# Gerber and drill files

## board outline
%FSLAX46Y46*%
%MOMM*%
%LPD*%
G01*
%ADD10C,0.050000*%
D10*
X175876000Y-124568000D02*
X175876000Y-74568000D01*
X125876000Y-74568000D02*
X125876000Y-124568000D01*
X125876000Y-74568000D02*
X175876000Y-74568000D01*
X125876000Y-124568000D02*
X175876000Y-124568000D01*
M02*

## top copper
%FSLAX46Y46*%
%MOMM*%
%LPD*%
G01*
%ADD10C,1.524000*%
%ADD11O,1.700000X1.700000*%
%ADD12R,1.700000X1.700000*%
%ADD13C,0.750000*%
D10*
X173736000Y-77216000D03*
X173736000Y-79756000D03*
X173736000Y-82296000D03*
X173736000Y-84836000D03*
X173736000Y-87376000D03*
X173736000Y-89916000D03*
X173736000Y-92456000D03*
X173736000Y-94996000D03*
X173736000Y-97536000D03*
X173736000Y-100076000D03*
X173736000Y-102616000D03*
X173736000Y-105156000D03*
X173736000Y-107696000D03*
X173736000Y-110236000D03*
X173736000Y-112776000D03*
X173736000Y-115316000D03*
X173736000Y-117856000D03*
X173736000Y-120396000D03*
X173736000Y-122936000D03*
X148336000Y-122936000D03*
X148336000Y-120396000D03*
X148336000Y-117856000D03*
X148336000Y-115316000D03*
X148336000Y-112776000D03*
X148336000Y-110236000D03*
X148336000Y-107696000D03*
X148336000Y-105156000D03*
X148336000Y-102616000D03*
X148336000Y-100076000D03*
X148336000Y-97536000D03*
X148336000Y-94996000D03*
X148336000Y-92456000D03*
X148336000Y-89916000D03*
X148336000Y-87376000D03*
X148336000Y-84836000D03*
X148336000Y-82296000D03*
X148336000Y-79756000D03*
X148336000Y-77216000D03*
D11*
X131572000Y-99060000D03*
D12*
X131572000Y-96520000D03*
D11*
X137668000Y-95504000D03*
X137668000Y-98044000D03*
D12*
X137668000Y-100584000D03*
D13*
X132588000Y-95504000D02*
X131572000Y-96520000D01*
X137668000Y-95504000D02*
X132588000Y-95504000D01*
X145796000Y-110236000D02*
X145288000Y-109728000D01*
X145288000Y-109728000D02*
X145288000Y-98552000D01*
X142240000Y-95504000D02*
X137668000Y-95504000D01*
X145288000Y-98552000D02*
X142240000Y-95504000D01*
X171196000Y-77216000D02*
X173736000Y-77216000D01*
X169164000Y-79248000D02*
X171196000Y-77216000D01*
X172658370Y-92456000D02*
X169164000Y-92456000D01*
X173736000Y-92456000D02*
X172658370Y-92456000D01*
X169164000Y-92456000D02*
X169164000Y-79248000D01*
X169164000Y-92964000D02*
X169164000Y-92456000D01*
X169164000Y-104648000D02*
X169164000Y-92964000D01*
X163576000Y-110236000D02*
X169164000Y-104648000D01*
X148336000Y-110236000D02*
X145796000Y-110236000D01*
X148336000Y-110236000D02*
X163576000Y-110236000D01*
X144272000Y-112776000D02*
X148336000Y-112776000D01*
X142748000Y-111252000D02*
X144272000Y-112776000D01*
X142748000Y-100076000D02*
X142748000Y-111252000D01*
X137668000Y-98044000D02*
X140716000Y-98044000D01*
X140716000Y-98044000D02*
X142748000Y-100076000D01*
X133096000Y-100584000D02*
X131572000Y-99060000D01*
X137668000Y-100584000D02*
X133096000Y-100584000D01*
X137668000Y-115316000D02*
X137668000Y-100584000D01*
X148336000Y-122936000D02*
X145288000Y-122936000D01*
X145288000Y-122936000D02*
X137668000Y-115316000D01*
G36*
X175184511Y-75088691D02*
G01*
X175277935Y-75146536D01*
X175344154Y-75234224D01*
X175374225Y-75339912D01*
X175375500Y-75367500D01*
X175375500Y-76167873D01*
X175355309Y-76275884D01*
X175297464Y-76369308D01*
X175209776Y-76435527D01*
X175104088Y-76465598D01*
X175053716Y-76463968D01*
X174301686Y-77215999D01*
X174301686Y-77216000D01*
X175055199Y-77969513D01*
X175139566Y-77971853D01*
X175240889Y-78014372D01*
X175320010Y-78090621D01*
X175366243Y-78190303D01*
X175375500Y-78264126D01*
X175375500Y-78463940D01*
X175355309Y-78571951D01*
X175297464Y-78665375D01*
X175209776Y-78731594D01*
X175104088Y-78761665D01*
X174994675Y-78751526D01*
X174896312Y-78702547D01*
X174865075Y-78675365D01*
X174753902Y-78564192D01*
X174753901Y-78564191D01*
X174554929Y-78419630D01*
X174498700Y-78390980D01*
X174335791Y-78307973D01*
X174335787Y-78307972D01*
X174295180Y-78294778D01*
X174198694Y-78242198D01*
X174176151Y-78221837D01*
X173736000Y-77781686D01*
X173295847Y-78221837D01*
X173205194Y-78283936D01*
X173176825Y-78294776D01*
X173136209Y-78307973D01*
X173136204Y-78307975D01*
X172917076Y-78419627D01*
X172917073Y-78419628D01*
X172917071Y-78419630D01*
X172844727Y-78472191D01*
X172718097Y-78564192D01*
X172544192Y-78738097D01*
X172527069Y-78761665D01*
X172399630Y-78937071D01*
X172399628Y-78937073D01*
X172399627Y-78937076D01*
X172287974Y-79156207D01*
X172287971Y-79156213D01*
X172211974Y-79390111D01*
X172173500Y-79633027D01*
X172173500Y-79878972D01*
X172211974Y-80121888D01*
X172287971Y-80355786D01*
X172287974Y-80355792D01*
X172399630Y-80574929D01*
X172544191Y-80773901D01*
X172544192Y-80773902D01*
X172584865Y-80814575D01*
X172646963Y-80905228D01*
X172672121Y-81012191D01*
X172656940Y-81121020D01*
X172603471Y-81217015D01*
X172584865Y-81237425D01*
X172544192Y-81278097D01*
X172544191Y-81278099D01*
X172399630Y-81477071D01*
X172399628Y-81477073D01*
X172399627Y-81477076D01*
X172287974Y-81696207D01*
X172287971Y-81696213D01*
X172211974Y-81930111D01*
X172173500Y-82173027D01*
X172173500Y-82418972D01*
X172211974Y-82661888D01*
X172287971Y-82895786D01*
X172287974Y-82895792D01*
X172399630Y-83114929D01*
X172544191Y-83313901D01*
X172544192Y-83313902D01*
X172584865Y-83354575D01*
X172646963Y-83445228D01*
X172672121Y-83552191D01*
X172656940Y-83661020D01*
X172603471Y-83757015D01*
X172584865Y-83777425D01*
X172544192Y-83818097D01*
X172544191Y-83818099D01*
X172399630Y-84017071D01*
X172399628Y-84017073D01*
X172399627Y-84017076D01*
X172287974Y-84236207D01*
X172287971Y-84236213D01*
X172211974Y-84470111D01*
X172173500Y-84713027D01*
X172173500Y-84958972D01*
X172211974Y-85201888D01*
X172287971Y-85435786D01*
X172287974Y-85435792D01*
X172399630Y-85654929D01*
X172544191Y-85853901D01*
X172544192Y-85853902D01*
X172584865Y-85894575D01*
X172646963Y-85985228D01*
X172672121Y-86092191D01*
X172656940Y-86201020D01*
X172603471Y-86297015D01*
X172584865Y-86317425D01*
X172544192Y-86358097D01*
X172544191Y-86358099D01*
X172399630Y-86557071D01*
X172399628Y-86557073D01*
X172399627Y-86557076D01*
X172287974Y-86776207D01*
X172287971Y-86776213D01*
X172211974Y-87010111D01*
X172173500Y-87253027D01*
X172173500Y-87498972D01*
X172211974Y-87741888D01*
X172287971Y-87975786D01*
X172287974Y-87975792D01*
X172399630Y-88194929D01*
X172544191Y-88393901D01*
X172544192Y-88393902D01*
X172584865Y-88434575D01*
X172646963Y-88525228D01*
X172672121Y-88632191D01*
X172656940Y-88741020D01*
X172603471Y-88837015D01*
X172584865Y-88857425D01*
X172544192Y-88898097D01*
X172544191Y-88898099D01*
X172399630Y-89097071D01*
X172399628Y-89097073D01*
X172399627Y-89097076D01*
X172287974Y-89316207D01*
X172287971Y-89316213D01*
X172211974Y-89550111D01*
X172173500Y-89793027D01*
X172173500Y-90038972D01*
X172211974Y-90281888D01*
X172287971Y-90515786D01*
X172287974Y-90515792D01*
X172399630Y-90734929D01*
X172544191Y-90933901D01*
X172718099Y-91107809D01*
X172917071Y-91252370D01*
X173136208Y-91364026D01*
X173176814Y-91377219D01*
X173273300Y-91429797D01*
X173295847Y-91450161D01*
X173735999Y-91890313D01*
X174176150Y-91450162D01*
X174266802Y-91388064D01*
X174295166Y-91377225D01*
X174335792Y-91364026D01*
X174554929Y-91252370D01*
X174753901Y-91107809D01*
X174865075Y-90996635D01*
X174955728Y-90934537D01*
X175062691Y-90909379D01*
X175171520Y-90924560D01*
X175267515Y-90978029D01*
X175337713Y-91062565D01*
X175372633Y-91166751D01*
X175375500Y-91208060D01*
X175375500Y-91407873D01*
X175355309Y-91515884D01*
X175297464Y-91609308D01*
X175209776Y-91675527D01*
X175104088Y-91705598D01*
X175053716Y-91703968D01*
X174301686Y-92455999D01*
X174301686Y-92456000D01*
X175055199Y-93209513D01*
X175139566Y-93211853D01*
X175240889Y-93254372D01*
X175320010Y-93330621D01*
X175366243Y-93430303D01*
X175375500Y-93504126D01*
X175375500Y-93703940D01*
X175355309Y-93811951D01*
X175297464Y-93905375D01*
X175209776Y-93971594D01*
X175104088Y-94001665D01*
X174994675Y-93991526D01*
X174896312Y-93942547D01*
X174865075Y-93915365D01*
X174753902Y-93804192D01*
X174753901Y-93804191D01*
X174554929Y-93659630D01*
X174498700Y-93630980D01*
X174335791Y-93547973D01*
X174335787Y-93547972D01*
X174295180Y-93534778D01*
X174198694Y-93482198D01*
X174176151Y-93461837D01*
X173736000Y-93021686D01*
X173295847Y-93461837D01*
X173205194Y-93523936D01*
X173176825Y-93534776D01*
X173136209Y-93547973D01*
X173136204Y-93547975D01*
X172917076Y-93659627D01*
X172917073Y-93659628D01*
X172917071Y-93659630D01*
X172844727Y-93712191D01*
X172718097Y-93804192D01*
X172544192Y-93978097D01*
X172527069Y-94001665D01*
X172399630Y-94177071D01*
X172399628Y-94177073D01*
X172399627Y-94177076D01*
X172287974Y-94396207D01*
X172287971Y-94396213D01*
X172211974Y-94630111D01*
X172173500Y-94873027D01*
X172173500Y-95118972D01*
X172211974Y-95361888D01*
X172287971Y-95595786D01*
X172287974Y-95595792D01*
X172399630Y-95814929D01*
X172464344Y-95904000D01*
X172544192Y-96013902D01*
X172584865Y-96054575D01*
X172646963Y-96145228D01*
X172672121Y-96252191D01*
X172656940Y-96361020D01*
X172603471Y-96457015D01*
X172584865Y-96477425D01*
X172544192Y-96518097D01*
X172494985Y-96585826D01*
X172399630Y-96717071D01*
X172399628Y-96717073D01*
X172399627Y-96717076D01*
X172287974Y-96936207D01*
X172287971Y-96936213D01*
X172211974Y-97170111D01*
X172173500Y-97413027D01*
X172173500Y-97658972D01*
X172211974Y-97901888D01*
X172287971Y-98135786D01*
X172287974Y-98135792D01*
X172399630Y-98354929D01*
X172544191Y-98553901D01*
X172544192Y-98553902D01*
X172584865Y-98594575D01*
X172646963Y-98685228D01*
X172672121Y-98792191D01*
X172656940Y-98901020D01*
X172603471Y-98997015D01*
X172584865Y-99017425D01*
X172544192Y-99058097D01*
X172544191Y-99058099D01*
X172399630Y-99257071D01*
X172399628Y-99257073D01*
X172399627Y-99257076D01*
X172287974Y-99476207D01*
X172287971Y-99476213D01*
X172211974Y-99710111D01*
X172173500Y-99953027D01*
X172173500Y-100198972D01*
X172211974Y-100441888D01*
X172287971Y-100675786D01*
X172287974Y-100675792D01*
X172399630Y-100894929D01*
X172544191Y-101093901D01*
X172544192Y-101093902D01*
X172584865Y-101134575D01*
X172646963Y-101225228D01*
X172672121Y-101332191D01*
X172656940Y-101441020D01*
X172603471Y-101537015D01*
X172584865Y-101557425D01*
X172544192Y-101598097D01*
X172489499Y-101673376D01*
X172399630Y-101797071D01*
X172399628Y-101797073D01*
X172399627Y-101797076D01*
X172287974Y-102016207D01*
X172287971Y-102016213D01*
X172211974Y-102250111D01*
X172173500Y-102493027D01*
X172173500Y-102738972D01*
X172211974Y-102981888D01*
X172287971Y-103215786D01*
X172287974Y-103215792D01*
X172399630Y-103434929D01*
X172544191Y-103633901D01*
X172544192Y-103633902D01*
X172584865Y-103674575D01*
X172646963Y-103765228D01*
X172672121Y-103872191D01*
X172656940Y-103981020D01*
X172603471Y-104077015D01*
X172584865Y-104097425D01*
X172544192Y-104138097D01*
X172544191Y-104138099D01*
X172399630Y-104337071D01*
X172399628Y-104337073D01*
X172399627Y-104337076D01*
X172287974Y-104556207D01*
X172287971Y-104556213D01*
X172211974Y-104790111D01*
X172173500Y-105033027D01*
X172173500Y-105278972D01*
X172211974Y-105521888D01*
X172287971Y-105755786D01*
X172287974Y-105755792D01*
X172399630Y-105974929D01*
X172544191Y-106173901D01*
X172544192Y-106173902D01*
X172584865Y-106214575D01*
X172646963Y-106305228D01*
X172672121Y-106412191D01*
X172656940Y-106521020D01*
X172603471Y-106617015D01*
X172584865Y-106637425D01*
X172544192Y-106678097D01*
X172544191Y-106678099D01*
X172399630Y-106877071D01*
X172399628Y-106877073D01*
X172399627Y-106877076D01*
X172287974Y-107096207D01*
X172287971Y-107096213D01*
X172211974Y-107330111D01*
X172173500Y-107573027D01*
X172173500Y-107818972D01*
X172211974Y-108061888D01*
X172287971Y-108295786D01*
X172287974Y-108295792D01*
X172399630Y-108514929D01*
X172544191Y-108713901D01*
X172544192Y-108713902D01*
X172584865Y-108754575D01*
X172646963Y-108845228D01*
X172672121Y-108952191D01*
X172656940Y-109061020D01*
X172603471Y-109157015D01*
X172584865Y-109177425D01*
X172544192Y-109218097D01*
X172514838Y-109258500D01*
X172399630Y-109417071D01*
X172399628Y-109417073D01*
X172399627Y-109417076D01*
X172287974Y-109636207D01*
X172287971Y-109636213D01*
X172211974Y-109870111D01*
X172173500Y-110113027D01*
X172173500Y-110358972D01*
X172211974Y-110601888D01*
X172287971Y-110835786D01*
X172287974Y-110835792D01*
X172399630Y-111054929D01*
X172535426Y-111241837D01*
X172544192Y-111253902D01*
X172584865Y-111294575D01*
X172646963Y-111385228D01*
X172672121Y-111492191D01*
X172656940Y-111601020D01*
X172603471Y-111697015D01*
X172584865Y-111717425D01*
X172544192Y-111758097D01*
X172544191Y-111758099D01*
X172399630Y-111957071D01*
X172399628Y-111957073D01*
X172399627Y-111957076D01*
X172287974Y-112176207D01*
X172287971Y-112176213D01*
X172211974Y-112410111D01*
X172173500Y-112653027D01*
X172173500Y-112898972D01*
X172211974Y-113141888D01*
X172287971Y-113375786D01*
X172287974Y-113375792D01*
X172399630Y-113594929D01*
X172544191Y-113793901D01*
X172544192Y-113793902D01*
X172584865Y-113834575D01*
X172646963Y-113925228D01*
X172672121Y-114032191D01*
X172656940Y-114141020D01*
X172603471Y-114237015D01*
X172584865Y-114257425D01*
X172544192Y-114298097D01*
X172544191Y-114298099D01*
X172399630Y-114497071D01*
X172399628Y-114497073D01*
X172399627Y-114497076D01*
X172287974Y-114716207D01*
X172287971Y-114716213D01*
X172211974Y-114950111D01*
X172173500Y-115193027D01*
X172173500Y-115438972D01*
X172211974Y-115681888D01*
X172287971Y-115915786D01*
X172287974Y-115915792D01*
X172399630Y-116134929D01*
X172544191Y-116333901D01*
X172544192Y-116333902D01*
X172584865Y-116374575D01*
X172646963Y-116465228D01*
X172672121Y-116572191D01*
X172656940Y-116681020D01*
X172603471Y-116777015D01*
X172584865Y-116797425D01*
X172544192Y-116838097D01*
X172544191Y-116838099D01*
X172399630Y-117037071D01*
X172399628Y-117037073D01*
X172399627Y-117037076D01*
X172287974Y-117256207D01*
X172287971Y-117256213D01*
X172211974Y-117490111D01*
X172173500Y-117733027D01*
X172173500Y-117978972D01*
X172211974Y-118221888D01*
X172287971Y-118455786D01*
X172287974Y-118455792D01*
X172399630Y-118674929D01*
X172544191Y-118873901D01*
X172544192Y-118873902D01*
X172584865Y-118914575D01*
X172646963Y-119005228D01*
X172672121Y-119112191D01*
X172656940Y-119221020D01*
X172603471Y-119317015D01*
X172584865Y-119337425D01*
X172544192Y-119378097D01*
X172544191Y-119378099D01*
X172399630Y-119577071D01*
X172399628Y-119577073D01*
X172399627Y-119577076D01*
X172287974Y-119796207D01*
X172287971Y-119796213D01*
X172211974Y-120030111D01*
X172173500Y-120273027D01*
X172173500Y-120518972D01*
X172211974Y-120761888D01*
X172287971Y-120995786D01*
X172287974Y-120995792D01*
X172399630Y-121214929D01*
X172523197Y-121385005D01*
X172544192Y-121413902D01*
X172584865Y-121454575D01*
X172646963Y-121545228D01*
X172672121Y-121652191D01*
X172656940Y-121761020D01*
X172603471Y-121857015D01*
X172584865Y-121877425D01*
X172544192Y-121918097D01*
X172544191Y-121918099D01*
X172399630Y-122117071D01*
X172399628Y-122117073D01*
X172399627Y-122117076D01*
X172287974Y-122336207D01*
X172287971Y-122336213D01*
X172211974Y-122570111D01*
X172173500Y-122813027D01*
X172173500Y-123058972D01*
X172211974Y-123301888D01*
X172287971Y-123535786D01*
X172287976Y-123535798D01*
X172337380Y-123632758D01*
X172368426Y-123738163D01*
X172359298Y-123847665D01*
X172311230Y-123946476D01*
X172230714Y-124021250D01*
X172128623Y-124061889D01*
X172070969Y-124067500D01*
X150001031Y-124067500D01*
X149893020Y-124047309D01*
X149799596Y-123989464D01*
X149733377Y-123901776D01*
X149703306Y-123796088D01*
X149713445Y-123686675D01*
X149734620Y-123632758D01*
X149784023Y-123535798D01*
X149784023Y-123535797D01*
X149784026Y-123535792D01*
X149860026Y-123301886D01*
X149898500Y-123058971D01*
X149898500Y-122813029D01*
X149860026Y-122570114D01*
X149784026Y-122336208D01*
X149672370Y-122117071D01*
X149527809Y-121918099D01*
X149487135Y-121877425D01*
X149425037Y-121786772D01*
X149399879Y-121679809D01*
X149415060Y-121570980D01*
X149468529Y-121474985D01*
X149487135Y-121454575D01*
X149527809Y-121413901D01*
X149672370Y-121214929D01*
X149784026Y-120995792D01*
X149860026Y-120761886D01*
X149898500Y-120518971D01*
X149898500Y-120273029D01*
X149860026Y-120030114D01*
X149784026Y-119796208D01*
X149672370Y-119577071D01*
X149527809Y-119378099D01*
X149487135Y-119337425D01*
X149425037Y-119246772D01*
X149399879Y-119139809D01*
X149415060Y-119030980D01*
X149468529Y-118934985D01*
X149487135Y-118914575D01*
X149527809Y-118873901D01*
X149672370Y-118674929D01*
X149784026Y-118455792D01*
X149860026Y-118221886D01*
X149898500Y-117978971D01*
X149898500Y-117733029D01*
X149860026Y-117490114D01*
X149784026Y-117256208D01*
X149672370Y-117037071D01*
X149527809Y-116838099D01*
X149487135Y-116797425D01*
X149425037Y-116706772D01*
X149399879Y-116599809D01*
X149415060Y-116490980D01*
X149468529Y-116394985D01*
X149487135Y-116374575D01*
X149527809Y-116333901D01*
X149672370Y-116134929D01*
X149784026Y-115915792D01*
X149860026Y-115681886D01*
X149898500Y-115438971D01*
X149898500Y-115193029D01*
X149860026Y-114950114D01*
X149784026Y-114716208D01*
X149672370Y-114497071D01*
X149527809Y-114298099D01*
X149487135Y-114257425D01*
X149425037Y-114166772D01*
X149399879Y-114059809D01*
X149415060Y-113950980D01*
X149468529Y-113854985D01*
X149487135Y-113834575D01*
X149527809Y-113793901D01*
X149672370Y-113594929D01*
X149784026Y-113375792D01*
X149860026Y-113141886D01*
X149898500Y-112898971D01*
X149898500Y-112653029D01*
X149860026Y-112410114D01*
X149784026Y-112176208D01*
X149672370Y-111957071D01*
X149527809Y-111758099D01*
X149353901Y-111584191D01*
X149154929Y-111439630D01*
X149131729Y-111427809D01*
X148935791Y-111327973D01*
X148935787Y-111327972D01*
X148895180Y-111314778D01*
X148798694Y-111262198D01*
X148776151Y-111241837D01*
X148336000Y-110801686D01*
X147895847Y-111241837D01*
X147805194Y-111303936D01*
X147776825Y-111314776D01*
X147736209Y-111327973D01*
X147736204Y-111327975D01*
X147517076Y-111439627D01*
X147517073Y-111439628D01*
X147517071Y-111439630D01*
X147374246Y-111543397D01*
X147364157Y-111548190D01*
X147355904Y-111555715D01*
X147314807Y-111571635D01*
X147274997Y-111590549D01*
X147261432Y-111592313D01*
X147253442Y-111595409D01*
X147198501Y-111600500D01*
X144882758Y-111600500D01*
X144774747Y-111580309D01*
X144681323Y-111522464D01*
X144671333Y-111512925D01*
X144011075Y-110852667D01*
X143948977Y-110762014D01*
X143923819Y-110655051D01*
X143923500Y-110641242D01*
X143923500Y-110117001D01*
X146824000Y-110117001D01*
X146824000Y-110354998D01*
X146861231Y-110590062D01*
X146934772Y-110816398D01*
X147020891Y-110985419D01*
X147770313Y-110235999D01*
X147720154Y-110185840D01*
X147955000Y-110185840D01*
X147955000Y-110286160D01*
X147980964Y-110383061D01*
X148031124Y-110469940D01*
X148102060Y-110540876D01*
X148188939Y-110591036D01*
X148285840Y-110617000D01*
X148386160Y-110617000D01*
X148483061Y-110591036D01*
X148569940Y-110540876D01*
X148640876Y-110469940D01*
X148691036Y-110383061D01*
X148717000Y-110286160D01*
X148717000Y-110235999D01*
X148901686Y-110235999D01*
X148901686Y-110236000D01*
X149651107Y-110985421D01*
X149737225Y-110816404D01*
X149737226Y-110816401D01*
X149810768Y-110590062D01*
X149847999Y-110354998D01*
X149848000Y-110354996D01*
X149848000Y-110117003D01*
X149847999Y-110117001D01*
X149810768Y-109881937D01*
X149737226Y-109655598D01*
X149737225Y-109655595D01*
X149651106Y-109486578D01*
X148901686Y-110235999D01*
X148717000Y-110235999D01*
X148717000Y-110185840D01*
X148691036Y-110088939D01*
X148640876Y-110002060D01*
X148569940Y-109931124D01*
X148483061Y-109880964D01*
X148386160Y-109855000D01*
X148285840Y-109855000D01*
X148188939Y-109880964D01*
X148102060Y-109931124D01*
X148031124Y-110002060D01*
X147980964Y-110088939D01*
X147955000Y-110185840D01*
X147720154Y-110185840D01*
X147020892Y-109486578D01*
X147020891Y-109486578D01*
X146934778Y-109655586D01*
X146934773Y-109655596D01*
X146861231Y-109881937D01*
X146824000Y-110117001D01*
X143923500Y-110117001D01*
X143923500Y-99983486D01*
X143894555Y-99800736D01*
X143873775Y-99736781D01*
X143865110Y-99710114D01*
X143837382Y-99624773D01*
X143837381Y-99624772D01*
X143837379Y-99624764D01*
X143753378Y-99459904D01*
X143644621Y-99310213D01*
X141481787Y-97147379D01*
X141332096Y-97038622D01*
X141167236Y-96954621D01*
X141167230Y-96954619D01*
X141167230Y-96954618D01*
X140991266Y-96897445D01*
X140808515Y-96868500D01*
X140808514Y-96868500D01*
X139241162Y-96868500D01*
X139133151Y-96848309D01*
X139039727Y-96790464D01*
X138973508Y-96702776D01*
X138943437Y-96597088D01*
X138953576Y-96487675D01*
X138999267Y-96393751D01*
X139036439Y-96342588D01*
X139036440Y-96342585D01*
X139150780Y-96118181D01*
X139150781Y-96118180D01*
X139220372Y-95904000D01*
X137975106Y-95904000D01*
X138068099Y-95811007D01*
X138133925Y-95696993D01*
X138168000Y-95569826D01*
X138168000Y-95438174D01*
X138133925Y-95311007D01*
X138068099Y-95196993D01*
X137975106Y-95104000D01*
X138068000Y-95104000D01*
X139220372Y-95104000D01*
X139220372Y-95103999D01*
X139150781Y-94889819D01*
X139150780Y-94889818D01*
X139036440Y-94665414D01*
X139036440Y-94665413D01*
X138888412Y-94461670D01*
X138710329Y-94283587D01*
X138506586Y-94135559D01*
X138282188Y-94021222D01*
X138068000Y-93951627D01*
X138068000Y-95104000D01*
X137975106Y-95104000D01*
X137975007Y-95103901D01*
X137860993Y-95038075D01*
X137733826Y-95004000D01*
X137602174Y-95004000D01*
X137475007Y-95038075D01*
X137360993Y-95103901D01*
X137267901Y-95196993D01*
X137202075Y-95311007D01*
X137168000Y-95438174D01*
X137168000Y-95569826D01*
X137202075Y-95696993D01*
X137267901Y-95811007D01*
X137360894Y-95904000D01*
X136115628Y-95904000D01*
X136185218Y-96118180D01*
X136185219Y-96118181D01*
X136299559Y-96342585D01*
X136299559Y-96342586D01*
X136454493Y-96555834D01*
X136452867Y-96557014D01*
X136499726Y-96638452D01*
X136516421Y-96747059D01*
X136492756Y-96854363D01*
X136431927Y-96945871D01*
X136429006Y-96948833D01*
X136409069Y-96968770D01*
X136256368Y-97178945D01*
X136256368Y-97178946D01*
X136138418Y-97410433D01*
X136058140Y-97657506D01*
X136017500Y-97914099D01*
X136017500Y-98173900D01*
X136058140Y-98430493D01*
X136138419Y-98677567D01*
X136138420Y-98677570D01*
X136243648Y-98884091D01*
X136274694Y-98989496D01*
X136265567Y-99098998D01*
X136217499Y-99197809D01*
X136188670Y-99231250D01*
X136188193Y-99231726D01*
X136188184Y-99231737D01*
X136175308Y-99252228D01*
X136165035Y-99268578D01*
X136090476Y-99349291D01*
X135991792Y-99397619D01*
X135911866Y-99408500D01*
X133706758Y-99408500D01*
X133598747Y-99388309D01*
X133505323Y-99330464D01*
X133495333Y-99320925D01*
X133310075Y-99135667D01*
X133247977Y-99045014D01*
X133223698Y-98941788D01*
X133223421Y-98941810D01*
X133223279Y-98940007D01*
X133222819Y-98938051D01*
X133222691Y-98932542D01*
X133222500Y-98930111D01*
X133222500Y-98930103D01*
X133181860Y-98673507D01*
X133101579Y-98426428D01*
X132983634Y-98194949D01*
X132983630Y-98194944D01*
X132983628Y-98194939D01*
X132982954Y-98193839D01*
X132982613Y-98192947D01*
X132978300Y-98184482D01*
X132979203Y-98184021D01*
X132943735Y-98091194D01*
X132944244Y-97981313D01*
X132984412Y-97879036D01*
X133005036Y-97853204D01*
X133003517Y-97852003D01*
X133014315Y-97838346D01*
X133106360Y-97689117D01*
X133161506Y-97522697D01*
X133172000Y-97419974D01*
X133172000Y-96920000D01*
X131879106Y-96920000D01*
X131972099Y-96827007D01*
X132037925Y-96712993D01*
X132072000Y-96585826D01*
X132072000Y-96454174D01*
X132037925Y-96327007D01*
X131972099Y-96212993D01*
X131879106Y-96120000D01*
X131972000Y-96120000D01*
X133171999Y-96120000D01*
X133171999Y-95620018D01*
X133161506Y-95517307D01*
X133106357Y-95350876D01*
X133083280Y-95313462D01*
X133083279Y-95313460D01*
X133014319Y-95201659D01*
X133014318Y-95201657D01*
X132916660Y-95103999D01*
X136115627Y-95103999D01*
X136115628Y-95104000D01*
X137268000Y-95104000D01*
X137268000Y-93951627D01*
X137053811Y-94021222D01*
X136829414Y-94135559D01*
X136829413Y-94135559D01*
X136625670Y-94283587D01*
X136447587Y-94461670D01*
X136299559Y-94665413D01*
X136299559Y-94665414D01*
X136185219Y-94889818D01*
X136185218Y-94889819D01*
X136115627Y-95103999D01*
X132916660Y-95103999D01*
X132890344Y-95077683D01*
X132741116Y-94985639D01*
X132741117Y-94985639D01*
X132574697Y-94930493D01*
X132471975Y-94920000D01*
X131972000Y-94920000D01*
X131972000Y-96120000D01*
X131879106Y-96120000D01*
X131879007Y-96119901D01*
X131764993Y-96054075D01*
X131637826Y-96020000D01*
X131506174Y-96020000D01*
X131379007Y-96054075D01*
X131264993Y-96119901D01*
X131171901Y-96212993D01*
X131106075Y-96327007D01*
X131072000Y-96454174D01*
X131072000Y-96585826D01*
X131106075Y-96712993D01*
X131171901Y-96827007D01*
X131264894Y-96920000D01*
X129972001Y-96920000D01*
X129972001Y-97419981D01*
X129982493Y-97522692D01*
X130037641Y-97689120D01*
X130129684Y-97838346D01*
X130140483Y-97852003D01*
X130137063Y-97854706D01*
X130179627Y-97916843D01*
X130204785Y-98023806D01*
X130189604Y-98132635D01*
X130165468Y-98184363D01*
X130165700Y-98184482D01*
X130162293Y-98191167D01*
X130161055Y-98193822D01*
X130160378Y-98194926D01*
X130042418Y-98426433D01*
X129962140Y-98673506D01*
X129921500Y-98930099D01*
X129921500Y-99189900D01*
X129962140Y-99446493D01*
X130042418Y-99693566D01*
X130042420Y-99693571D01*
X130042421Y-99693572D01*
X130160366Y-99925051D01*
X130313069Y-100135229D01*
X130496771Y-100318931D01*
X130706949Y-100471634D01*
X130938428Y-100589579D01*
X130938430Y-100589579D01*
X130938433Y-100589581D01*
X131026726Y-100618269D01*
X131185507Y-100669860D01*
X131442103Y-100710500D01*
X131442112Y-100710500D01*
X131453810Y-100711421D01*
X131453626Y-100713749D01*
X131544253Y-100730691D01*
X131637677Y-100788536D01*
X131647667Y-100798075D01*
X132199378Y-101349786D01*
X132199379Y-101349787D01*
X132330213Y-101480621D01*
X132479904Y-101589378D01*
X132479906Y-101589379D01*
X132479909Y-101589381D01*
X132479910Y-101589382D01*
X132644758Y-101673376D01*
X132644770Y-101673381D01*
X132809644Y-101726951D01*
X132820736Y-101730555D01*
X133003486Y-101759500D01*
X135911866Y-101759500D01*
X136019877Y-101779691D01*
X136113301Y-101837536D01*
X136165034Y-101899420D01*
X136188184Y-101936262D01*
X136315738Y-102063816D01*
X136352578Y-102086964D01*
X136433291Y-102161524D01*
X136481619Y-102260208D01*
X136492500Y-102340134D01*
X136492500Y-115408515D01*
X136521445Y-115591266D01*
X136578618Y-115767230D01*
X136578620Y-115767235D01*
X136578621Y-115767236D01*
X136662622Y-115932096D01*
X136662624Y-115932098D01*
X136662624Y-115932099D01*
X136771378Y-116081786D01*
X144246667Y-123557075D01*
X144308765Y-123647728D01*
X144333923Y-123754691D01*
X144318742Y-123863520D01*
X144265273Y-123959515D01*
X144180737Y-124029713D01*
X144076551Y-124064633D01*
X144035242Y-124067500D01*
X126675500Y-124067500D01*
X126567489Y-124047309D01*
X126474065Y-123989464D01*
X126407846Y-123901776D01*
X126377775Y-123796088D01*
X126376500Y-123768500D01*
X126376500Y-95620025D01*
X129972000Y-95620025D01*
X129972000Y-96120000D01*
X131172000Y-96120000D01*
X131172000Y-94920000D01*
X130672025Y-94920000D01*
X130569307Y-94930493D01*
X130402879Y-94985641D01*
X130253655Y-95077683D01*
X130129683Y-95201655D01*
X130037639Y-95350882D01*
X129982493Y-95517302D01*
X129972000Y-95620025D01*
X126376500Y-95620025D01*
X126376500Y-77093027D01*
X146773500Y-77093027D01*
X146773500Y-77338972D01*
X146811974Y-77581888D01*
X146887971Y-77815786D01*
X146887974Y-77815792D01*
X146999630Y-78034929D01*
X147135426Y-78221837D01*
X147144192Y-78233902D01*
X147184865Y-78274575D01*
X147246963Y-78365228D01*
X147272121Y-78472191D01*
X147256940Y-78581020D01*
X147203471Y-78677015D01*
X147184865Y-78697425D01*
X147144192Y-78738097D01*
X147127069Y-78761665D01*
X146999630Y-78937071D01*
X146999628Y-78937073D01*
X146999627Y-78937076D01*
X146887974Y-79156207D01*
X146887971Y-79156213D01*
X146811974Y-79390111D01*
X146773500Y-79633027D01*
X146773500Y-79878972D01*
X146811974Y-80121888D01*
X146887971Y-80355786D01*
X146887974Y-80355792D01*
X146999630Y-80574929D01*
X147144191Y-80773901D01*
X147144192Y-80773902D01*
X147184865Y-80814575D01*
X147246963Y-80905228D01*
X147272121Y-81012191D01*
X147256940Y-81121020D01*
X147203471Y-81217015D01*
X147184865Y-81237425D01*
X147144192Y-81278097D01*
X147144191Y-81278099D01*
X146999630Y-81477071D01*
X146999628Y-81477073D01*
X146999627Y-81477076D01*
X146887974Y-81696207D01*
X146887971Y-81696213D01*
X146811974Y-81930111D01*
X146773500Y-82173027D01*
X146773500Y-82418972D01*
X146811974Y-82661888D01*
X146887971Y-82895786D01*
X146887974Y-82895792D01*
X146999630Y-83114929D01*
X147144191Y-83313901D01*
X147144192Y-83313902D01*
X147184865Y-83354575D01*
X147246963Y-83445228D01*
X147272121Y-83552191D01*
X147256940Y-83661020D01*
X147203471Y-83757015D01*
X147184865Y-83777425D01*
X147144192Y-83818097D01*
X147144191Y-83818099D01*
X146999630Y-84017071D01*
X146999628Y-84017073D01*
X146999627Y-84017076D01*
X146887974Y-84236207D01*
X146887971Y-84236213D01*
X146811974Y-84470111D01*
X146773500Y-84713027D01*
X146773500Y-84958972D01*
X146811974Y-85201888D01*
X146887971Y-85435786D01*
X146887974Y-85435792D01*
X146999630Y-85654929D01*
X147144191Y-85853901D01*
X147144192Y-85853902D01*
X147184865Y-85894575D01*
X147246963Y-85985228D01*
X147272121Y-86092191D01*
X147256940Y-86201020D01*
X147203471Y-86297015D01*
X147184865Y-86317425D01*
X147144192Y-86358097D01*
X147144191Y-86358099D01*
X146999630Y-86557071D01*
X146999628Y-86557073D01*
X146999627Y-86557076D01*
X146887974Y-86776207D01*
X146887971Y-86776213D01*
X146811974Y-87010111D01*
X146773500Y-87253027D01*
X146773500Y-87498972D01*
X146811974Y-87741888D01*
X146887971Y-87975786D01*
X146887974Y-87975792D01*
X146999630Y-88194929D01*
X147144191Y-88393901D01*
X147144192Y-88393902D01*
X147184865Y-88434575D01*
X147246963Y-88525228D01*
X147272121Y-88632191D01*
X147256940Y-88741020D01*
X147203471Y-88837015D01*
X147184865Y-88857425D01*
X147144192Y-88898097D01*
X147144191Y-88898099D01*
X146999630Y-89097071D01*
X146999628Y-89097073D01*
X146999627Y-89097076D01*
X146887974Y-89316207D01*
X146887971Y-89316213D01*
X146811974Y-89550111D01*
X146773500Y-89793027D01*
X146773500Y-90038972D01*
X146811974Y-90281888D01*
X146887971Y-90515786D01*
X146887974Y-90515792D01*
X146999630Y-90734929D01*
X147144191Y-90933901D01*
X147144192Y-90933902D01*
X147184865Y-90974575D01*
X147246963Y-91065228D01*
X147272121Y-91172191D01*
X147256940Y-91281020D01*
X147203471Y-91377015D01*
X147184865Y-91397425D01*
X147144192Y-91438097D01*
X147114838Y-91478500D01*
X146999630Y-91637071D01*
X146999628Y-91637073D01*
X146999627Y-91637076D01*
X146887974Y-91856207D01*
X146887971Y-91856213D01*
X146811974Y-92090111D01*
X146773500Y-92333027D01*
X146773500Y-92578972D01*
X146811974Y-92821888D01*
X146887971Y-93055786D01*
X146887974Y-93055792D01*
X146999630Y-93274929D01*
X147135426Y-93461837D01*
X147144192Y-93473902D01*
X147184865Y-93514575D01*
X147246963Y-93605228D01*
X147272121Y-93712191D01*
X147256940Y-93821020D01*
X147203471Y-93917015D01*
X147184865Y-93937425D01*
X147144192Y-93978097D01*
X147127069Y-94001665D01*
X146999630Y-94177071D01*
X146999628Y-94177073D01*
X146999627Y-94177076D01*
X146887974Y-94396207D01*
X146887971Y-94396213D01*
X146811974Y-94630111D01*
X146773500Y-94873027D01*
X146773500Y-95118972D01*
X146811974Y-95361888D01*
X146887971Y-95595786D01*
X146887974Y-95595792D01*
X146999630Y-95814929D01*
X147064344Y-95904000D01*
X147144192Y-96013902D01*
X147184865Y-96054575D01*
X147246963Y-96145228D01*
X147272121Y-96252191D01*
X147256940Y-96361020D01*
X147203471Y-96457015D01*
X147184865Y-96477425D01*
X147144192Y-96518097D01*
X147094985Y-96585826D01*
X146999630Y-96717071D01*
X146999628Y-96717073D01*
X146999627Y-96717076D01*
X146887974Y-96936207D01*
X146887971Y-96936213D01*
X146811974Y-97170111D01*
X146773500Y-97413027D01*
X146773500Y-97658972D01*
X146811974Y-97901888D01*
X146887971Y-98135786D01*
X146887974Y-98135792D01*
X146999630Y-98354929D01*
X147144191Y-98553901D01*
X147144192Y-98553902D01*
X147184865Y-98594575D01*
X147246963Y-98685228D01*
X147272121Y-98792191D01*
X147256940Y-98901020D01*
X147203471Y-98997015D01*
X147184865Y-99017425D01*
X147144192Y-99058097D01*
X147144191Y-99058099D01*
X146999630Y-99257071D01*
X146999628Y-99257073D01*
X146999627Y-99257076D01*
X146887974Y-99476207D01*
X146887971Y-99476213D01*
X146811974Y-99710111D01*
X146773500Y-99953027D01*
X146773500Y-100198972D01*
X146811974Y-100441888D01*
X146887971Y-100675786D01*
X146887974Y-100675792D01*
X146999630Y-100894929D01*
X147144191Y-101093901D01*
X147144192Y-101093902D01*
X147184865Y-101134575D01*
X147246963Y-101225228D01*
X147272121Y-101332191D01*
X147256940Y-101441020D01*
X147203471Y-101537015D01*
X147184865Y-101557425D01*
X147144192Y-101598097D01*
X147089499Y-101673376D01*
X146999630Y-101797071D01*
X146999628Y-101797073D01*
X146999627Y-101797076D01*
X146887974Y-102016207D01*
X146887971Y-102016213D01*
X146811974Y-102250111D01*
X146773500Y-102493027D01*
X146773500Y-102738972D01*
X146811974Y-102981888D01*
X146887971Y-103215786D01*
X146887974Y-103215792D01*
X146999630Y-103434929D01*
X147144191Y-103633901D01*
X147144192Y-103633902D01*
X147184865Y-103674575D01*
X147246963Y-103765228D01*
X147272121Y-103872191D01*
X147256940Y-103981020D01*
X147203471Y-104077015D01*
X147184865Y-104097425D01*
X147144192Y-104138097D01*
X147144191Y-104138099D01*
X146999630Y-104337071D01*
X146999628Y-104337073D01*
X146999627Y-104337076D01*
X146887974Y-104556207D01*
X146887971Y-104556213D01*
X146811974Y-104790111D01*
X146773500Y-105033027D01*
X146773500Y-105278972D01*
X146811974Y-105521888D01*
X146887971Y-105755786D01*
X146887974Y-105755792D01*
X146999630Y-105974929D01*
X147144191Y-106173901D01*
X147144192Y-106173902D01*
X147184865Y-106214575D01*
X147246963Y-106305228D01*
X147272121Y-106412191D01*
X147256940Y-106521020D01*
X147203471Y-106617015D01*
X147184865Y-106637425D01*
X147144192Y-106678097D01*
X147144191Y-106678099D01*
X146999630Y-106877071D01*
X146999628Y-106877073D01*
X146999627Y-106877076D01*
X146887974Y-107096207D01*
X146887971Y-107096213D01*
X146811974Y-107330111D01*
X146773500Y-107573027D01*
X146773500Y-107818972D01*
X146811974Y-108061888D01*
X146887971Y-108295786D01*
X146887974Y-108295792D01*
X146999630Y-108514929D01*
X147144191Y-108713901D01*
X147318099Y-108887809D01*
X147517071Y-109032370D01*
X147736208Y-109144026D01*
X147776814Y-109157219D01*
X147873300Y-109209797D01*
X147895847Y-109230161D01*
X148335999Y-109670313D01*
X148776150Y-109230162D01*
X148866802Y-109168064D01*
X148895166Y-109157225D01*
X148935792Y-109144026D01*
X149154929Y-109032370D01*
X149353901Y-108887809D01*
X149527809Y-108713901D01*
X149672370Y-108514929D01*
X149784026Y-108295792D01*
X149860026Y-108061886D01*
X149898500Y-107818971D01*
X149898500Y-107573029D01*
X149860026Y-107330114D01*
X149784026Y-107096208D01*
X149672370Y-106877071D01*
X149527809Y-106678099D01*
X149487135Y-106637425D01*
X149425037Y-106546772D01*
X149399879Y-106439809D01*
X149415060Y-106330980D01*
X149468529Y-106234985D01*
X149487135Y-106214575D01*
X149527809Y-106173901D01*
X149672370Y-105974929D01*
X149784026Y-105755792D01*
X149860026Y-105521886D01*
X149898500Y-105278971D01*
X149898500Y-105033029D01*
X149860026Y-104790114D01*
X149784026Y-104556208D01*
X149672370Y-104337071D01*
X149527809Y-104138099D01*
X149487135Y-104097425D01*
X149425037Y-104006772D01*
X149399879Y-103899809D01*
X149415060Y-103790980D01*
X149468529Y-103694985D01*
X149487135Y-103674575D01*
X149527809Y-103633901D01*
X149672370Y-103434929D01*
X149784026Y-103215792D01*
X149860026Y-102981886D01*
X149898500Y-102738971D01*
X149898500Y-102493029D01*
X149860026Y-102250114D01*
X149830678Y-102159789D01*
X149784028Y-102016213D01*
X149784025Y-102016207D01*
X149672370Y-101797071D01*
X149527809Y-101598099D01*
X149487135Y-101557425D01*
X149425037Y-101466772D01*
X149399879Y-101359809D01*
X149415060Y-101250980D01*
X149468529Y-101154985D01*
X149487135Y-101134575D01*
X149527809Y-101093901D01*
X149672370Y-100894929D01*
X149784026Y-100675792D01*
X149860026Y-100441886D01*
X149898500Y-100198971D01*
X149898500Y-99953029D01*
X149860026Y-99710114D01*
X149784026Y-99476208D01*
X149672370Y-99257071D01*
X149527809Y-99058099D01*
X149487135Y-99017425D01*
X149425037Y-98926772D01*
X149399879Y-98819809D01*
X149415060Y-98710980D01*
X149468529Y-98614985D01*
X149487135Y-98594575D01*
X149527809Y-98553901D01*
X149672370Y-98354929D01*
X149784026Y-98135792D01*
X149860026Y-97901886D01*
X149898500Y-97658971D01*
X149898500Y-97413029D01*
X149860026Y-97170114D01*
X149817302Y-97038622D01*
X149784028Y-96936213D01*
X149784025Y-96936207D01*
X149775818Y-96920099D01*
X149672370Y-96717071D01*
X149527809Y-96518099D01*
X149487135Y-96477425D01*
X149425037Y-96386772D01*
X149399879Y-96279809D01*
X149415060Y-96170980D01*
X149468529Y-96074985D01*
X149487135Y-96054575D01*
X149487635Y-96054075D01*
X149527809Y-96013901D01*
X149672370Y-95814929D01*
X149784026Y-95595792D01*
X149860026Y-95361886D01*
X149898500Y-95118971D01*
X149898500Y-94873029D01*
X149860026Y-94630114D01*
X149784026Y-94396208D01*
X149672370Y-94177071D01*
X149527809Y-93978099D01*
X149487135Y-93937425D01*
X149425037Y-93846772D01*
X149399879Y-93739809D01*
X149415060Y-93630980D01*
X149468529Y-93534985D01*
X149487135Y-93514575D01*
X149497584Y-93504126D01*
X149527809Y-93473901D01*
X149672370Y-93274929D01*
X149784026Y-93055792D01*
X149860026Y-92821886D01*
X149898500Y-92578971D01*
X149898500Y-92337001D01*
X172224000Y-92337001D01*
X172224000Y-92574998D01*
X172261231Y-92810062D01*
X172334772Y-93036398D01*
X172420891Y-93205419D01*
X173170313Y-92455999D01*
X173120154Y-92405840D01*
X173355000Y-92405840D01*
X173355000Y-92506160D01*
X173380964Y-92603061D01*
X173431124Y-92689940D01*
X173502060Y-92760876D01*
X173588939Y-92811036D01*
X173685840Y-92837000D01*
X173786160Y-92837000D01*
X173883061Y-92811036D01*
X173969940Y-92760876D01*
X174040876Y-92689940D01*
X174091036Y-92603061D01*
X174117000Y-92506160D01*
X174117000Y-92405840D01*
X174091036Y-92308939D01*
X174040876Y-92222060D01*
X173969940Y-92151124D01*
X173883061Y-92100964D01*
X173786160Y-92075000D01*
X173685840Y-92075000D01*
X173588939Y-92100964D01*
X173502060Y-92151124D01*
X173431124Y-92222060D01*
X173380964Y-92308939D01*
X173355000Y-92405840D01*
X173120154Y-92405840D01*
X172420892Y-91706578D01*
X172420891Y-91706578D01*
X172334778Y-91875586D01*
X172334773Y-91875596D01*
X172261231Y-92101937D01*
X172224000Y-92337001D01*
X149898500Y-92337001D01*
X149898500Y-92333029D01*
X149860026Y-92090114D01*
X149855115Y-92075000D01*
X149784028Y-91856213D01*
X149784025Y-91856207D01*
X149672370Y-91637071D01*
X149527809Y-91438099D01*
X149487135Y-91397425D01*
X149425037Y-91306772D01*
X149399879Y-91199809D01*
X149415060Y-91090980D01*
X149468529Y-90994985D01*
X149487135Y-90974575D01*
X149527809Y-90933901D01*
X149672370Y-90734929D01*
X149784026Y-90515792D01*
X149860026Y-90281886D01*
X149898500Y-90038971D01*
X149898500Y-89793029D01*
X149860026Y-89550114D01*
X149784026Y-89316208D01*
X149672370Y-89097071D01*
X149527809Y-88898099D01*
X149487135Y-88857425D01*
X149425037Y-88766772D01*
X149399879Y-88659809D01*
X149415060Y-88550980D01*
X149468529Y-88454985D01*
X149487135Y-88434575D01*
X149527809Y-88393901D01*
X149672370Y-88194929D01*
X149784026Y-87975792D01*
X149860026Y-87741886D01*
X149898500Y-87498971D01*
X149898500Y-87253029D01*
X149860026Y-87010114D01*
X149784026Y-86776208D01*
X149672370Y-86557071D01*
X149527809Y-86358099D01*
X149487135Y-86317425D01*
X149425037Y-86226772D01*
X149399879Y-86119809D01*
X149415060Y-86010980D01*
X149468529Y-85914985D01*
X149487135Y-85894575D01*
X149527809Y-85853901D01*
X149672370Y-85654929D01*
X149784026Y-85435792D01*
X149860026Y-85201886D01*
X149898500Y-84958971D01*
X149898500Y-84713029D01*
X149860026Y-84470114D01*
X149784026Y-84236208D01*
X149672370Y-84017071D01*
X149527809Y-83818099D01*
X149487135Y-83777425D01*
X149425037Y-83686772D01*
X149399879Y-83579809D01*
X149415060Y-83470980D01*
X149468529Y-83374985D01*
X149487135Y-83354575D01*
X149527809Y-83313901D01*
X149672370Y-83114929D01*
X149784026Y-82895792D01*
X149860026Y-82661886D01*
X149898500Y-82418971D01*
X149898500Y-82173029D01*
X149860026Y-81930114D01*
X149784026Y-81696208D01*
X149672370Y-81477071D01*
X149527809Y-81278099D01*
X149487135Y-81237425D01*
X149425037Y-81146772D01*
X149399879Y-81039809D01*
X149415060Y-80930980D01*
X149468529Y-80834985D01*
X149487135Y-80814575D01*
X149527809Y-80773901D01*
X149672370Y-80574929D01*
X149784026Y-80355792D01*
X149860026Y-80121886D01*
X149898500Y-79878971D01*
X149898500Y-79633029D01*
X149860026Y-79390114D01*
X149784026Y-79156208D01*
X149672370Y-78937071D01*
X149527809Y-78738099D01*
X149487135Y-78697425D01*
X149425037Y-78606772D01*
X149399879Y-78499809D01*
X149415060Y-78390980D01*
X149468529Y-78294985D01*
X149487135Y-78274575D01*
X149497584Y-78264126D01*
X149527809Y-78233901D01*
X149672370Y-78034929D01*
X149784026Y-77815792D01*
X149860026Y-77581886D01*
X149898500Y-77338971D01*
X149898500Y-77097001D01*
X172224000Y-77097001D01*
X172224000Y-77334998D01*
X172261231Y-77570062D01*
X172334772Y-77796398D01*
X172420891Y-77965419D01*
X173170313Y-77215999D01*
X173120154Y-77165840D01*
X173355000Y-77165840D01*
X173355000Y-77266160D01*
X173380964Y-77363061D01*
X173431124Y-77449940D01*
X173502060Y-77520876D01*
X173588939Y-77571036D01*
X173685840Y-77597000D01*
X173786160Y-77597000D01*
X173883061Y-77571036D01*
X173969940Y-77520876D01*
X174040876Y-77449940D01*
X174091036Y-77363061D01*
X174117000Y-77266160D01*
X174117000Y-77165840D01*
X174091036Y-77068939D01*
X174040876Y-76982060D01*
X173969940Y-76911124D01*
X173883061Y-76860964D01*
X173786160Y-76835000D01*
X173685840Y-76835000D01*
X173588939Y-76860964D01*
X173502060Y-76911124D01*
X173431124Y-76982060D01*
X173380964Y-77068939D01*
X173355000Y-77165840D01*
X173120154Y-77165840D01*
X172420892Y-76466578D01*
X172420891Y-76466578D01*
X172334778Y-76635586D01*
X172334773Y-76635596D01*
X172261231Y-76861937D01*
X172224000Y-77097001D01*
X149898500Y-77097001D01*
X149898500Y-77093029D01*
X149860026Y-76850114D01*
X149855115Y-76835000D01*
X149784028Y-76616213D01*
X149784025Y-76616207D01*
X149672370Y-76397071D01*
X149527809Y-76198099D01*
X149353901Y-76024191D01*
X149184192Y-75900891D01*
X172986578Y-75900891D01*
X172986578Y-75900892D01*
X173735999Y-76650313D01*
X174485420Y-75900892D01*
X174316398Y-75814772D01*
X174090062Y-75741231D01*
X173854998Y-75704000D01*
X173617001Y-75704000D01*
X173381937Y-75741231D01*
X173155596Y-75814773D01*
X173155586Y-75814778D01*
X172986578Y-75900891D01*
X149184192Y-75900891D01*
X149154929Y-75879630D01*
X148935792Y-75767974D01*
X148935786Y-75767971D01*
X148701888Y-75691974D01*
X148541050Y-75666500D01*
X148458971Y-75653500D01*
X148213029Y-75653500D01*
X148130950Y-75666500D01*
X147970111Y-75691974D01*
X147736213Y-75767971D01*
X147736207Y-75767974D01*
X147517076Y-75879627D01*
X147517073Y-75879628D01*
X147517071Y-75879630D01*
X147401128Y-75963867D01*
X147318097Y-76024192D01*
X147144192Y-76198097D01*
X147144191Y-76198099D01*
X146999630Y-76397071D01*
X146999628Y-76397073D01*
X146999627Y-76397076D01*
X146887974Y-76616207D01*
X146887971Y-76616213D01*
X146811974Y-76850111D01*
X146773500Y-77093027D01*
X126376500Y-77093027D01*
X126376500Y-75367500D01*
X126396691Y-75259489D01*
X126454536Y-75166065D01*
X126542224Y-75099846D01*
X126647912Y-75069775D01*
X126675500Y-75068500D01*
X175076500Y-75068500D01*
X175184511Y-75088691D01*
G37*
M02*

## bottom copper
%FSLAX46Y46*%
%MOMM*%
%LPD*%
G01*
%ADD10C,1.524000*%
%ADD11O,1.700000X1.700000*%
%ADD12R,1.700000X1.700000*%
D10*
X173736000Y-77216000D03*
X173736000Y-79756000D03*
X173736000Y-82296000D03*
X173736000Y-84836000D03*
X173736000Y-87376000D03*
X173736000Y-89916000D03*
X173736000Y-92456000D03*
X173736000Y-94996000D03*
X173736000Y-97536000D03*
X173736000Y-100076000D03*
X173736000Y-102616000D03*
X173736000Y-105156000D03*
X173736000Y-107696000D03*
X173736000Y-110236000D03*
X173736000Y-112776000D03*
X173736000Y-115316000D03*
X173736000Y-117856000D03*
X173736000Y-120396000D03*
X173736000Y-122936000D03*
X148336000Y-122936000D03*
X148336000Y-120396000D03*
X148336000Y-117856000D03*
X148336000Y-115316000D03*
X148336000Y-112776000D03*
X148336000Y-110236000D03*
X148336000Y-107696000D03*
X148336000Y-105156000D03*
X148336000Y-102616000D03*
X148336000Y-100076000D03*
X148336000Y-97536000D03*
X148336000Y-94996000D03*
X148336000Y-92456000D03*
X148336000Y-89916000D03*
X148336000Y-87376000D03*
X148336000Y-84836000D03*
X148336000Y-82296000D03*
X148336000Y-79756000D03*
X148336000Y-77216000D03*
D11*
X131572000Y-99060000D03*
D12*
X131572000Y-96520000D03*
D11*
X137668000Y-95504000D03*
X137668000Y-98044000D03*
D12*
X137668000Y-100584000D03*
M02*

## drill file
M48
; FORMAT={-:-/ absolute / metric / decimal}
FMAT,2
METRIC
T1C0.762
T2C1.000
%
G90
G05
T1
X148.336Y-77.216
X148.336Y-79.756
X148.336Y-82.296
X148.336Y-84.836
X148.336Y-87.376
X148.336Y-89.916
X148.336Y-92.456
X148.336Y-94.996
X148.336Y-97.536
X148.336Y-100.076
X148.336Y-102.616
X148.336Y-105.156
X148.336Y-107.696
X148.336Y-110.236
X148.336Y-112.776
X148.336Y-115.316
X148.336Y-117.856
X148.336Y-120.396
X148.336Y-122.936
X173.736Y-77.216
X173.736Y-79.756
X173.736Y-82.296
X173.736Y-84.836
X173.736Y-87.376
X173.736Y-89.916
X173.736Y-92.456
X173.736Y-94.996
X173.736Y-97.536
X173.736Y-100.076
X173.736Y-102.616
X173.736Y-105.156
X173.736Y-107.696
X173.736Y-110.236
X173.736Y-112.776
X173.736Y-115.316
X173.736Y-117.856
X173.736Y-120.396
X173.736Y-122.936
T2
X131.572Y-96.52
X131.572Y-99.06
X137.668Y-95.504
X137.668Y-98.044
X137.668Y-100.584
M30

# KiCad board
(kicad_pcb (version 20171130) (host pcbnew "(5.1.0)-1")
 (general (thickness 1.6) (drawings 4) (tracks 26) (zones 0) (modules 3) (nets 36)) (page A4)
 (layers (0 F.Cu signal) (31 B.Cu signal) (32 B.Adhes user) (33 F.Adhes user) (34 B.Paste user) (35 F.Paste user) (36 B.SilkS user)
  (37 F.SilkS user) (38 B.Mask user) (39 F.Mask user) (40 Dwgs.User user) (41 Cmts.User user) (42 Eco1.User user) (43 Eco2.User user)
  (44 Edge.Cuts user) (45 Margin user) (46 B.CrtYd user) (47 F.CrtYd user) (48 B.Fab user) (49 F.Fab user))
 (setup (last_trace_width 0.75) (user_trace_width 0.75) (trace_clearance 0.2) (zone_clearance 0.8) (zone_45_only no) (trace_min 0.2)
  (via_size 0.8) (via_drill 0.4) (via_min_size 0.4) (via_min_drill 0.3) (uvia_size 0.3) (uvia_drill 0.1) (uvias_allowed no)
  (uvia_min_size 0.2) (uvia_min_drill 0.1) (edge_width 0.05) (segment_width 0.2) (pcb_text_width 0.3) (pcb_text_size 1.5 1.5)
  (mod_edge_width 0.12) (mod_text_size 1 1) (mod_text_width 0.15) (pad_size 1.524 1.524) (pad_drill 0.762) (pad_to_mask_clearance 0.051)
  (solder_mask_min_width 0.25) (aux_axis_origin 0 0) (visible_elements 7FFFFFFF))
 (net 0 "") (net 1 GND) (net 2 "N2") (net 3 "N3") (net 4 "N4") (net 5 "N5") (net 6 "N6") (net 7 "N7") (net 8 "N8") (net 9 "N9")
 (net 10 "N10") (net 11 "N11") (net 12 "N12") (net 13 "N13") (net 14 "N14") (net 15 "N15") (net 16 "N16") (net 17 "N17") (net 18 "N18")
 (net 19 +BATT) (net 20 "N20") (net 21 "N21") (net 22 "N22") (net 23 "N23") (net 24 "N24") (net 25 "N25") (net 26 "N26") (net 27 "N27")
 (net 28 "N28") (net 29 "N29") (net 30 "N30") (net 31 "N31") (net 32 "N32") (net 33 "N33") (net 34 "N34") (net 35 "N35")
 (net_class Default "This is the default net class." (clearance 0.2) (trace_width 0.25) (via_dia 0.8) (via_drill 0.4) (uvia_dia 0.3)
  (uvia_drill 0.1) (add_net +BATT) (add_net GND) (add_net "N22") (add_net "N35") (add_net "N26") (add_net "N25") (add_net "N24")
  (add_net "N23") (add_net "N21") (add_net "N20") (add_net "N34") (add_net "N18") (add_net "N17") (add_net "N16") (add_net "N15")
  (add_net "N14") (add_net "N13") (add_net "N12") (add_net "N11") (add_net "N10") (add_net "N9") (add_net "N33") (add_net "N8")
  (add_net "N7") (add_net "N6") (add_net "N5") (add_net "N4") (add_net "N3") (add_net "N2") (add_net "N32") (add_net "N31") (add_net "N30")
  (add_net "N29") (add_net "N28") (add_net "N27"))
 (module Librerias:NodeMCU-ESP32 (layer F.Cu) (at 161.036 97.536)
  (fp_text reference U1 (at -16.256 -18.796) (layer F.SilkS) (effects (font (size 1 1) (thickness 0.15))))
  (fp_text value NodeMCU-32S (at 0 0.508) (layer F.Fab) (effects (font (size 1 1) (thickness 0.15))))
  (pad 38 thru_hole circle (at 12.7 -20.32) (size 1.524 1.524) (drill 0.762) (layers *.Cu *.Mask) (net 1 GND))
  (pad 37 thru_hole circle (at 12.7 -17.78) (size 1.524 1.524) (drill 0.762) (layers *.Cu *.Mask) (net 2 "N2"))
  (pad 36 thru_hole circle (at 12.7 -15.24) (size 1.524 1.524) (drill 0.762) (layers *.Cu *.Mask) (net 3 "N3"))
  (pad 35 thru_hole circle (at 12.7 -12.7) (size 1.524 1.524) (drill 0.762) (layers *.Cu *.Mask) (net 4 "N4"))
  (pad 34 thru_hole circle (at 12.7 -10.16) (size 1.524 1.524) (drill 0.762) (layers *.Cu *.Mask) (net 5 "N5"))
  (pad 33 thru_hole circle (at 12.7 -7.62) (size 1.524 1.524) (drill 0.762) (layers *.Cu *.Mask) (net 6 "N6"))
  (pad 32 thru_hole circle (at 12.7 -5.08) (size 1.524 1.524) (drill 0.762) (layers *.Cu *.Mask) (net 1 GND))
  (pad 31 thru_hole circle (at 12.7 -2.54) (size 1.524 1.524) (drill 0.762) (layers *.Cu *.Mask) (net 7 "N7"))
  (pad 30 thru_hole circle (at 12.7 0) (size 1.524 1.524) (drill 0.762) (layers *.Cu *.Mask) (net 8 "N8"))
  (pad 29 thru_hole circle (at 12.7 2.54) (size 1.524 1.524) (drill 0.762) (layers *.Cu *.Mask) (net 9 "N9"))
  (pad 28 thru_hole circle (at 12.7 5.08) (size 1.524 1.524) (drill 0.762) (layers *.Cu *.Mask) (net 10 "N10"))
  (pad 27 thru_hole circle (at 12.7 7.62) (size 1.524 1.524) (drill 0.762) (layers *.Cu *.Mask) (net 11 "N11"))
  (pad 26 thru_hole circle (at 12.7 10.16) (size 1.524 1.524) (drill 0.762) (layers *.Cu *.Mask) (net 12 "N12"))
  (pad 25 thru_hole circle (at 12.7 12.7) (size 1.524 1.524) (drill 0.762) (layers *.Cu *.Mask) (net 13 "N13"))
  (pad 24 thru_hole circle (at 12.7 15.24) (size 1.524 1.524) (drill 0.762) (layers *.Cu *.Mask) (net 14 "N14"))
  (pad 23 thru_hole circle (at 12.7 17.78) (size 1.524 1.524) (drill 0.762) (layers *.Cu *.Mask) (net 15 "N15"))
  (pad 22 thru_hole circle (at 12.7 20.32) (size 1.524 1.524) (drill 0.762) (layers *.Cu *.Mask) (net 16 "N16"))
  (pad 21 thru_hole circle (at 12.7 22.86) (size 1.524 1.524) (drill 0.762) (layers *.Cu *.Mask) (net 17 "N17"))
  (pad 20 thru_hole circle (at 12.7 25.4) (size 1.524 1.524) (drill 0.762) (layers *.Cu *.Mask) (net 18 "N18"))
  (pad 19 thru_hole circle (at -12.7 25.4) (size 1.524 1.524) (drill 0.762) (layers *.Cu *.Mask) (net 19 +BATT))
  (pad 18 thru_hole circle (at -12.7 22.86) (size 1.524 1.524) (drill 0.762) (layers *.Cu *.Mask) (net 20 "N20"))
  (pad 17 thru_hole circle (at -12.7 20.32) (size 1.524 1.524) (drill 0.762) (layers *.Cu *.Mask) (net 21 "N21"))
  (pad 16 thru_hole circle (at -12.7 17.78) (size 1.524 1.524) (drill 0.762) (layers *.Cu *.Mask))
  (pad 15 thru_hole circle (at -12.7 15.24) (size 1.524 1.524) (drill 0.762) (layers *.Cu *.Mask) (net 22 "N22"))
  (pad 14 thru_hole circle (at -12.7 12.7) (size 1.524 1.524) (drill 0.762) (layers *.Cu *.Mask) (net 1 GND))
  (pad 13 thru_hole circle (at -12.7 10.16) (size 1.524 1.524) (drill 0.762) (layers *.Cu *.Mask) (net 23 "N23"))
  (pad 12 thru_hole circle (at -12.7 7.62) (size 1.524 1.524) (drill 0.762) (layers *.Cu *.Mask) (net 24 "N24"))
  (pad 11 thru_hole circle (at -12.7 5.08) (size 1.524 1.524) (drill 0.762) (layers *.Cu *.Mask) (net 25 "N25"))
  (pad 10 thru_hole circle (at -12.7 2.54) (size 1.524 1.524) (drill 0.762) (layers *.Cu *.Mask) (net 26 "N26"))
  (pad 9 thru_hole circle (at -12.7 0) (size 1.524 1.524) (drill 0.762) (layers *.Cu *.Mask) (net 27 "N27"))
  (pad 8 thru_hole circle (at -12.7 -2.54) (size 1.524 1.524) (drill 0.762) (layers *.Cu *.Mask) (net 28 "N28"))
  (pad 7 thru_hole circle (at -12.7 -5.08) (size 1.524 1.524) (drill 0.762) (layers *.Cu *.Mask) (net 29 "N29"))
  (pad 6 thru_hole circle (at -12.7 -7.62) (size 1.524 1.524) (drill 0.762) (layers *.Cu *.Mask) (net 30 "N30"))
  (pad 5 thru_hole circle (at -12.7 -10.16) (size 1.524 1.524) (drill 0.762) (layers *.Cu *.Mask) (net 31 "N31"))
  (pad 4 thru_hole circle (at -12.7 -12.7) (size 1.524 1.524) (drill 0.762) (layers *.Cu *.Mask) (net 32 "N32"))
  (pad 3 thru_hole circle (at -12.7 -15.24) (size 1.524 1.524) (drill 0.762) (layers *.Cu *.Mask) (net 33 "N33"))
  (pad 2 thru_hole circle (at -12.7 -17.78) (size 1.524 1.524) (drill 0.762) (layers *.Cu *.Mask) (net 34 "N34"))
  (pad 1 thru_hole circle (at -12.7 -20.32) (size 1.524 1.524) (drill 0.762) (layers *.Cu *.Mask) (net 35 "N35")))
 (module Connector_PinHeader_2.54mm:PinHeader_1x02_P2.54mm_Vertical (layer F.Cu) (at 131.572 96.52)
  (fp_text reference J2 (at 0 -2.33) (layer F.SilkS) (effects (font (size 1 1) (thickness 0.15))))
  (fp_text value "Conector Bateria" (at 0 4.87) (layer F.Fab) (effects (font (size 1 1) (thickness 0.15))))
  (pad 2 thru_hole oval (at 0 2.54) (size 1.7 1.7) (drill 1) (layers *.Cu *.Mask) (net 19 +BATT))
  (pad 1 thru_hole rect (at 0 0) (size 1.7 1.7) (drill 1) (layers *.Cu *.Mask) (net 1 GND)))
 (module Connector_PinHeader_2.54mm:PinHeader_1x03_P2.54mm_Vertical (layer F.Cu) (at 137.668 100.584 180)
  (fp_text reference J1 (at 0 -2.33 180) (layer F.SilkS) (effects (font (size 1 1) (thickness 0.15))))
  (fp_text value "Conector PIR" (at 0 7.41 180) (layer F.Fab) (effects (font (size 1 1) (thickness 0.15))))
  (pad 3 thru_hole oval (at 0 5.08 180) (size 1.7 1.7) (drill 1) (layers *.Cu *.Mask) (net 1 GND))
  (pad 2 thru_hole oval (at 0 2.54 180) (size 1.7 1.7) (drill 1) (layers *.Cu *.Mask) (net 22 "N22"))
  (pad 1 thru_hole rect (at 0 0 180) (size 1.7 1.7) (drill 1) (layers *.Cu *.Mask) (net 19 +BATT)))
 (gr_line (start 175.876 124.568) (end 175.876 74.568) (layer Edge.Cuts) (width 0.05))
 (gr_line (start 125.876 74.568) (end 125.876 124.568) (layer Edge.Cuts) (width 0.05))
 (gr_line (start 125.876 74.568) (end 175.876 74.568) (layer Edge.Cuts) (width 0.05))
 (gr_line (start 125.876 124.568) (end 175.876 124.568) (layer Edge.Cuts) (width 0.05))
 (segment (start 132.588 95.504) (end 131.572 96.52) (width 0.75) (layer F.Cu) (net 1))
 (segment (start 137.668 95.504) (end 132.588 95.504) (width 0.75) (layer F.Cu) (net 1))
 (segment (start 145.796 110.236) (end 145.288 109.728) (width 0.75) (layer F.Cu) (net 1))
 (segment (start 145.288 109.728) (end 145.288 98.552) (width 0.75) (layer F.Cu) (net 1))
 (segment (start 142.24 95.504) (end 137.668 95.504) (width 0.75) (layer F.Cu) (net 1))
 (segment (start 145.288 98.552) (end 142.24 95.504) (width 0.75) (layer F.Cu) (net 1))
 (segment (start 171.196 77.216) (end 173.736 77.216) (width 0.75) (layer F.Cu) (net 1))
 (segment (start 169.164 79.248) (end 171.196 77.216) (width 0.75) (layer F.Cu) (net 1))
 (segment (start 172.65837 92.456) (end 169.164 92.456) (width 0.75) (layer F.Cu) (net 1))
 (segment (start 173.736 92.456) (end 172.65837 92.456) (width 0.75) (layer F.Cu) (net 1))
 (segment (start 169.164 92.456) (end 169.164 79.248) (width 0.75) (layer F.Cu) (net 1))
 (segment (start 169.164 92.964) (end 169.164 92.456) (width 0.75) (layer F.Cu) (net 1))
 (segment (start 169.164 104.648) (end 169.164 92.964) (width 0.75) (layer F.Cu) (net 1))
 (segment (start 163.576 110.236) (end 169.164 104.648) (width 0.75) (layer F.Cu) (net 1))
 (segment (start 148.336 110.236) (end 145.796 110.236) (width 0.75) (layer F.Cu) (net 1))
 (segment (start 148.336 110.236) (end 163.576 110.236) (width 0.75) (layer F.Cu) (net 1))
 (segment (start 144.272 112.776) (end 148.336 112.776) (width 0.75) (layer F.Cu) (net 22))
 (segment (start 142.748 111.252) (end 144.272 112.776) (width 0.75) (layer F.Cu) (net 22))
 (segment (start 142.748 100.076) (end 142.748 111.252) (width 0.75) (layer F.Cu) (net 22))
 (segment (start 137.668 98.044) (end 140.716 98.044) (width 0.75) (layer F.Cu) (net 22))
 (segment (start 140.716 98.044) (end 142.748 100.076) (width 0.75) (layer F.Cu) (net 22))
 (segment (start 133.096 100.584) (end 131.572 99.06) (width 0.75) (layer F.Cu) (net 19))
 (segment (start 137.668 100.584) (end 133.096 100.584) (width 0.75) (layer F.Cu) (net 19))
 (segment (start 137.668 115.316) (end 137.668 100.584) (width 0.75) (layer F.Cu) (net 19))
 (segment (start 148.336 122.936) (end 145.288 122.936) (width 0.75) (layer F.Cu) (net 19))
 (segment (start 145.288 122.936) (end 137.668 115.316) (width 0.75) (layer F.Cu) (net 19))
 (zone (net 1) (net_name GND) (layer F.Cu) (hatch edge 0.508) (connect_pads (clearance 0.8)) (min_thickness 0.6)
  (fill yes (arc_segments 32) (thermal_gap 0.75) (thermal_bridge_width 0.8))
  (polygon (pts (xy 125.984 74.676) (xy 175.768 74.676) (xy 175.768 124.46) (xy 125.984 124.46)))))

